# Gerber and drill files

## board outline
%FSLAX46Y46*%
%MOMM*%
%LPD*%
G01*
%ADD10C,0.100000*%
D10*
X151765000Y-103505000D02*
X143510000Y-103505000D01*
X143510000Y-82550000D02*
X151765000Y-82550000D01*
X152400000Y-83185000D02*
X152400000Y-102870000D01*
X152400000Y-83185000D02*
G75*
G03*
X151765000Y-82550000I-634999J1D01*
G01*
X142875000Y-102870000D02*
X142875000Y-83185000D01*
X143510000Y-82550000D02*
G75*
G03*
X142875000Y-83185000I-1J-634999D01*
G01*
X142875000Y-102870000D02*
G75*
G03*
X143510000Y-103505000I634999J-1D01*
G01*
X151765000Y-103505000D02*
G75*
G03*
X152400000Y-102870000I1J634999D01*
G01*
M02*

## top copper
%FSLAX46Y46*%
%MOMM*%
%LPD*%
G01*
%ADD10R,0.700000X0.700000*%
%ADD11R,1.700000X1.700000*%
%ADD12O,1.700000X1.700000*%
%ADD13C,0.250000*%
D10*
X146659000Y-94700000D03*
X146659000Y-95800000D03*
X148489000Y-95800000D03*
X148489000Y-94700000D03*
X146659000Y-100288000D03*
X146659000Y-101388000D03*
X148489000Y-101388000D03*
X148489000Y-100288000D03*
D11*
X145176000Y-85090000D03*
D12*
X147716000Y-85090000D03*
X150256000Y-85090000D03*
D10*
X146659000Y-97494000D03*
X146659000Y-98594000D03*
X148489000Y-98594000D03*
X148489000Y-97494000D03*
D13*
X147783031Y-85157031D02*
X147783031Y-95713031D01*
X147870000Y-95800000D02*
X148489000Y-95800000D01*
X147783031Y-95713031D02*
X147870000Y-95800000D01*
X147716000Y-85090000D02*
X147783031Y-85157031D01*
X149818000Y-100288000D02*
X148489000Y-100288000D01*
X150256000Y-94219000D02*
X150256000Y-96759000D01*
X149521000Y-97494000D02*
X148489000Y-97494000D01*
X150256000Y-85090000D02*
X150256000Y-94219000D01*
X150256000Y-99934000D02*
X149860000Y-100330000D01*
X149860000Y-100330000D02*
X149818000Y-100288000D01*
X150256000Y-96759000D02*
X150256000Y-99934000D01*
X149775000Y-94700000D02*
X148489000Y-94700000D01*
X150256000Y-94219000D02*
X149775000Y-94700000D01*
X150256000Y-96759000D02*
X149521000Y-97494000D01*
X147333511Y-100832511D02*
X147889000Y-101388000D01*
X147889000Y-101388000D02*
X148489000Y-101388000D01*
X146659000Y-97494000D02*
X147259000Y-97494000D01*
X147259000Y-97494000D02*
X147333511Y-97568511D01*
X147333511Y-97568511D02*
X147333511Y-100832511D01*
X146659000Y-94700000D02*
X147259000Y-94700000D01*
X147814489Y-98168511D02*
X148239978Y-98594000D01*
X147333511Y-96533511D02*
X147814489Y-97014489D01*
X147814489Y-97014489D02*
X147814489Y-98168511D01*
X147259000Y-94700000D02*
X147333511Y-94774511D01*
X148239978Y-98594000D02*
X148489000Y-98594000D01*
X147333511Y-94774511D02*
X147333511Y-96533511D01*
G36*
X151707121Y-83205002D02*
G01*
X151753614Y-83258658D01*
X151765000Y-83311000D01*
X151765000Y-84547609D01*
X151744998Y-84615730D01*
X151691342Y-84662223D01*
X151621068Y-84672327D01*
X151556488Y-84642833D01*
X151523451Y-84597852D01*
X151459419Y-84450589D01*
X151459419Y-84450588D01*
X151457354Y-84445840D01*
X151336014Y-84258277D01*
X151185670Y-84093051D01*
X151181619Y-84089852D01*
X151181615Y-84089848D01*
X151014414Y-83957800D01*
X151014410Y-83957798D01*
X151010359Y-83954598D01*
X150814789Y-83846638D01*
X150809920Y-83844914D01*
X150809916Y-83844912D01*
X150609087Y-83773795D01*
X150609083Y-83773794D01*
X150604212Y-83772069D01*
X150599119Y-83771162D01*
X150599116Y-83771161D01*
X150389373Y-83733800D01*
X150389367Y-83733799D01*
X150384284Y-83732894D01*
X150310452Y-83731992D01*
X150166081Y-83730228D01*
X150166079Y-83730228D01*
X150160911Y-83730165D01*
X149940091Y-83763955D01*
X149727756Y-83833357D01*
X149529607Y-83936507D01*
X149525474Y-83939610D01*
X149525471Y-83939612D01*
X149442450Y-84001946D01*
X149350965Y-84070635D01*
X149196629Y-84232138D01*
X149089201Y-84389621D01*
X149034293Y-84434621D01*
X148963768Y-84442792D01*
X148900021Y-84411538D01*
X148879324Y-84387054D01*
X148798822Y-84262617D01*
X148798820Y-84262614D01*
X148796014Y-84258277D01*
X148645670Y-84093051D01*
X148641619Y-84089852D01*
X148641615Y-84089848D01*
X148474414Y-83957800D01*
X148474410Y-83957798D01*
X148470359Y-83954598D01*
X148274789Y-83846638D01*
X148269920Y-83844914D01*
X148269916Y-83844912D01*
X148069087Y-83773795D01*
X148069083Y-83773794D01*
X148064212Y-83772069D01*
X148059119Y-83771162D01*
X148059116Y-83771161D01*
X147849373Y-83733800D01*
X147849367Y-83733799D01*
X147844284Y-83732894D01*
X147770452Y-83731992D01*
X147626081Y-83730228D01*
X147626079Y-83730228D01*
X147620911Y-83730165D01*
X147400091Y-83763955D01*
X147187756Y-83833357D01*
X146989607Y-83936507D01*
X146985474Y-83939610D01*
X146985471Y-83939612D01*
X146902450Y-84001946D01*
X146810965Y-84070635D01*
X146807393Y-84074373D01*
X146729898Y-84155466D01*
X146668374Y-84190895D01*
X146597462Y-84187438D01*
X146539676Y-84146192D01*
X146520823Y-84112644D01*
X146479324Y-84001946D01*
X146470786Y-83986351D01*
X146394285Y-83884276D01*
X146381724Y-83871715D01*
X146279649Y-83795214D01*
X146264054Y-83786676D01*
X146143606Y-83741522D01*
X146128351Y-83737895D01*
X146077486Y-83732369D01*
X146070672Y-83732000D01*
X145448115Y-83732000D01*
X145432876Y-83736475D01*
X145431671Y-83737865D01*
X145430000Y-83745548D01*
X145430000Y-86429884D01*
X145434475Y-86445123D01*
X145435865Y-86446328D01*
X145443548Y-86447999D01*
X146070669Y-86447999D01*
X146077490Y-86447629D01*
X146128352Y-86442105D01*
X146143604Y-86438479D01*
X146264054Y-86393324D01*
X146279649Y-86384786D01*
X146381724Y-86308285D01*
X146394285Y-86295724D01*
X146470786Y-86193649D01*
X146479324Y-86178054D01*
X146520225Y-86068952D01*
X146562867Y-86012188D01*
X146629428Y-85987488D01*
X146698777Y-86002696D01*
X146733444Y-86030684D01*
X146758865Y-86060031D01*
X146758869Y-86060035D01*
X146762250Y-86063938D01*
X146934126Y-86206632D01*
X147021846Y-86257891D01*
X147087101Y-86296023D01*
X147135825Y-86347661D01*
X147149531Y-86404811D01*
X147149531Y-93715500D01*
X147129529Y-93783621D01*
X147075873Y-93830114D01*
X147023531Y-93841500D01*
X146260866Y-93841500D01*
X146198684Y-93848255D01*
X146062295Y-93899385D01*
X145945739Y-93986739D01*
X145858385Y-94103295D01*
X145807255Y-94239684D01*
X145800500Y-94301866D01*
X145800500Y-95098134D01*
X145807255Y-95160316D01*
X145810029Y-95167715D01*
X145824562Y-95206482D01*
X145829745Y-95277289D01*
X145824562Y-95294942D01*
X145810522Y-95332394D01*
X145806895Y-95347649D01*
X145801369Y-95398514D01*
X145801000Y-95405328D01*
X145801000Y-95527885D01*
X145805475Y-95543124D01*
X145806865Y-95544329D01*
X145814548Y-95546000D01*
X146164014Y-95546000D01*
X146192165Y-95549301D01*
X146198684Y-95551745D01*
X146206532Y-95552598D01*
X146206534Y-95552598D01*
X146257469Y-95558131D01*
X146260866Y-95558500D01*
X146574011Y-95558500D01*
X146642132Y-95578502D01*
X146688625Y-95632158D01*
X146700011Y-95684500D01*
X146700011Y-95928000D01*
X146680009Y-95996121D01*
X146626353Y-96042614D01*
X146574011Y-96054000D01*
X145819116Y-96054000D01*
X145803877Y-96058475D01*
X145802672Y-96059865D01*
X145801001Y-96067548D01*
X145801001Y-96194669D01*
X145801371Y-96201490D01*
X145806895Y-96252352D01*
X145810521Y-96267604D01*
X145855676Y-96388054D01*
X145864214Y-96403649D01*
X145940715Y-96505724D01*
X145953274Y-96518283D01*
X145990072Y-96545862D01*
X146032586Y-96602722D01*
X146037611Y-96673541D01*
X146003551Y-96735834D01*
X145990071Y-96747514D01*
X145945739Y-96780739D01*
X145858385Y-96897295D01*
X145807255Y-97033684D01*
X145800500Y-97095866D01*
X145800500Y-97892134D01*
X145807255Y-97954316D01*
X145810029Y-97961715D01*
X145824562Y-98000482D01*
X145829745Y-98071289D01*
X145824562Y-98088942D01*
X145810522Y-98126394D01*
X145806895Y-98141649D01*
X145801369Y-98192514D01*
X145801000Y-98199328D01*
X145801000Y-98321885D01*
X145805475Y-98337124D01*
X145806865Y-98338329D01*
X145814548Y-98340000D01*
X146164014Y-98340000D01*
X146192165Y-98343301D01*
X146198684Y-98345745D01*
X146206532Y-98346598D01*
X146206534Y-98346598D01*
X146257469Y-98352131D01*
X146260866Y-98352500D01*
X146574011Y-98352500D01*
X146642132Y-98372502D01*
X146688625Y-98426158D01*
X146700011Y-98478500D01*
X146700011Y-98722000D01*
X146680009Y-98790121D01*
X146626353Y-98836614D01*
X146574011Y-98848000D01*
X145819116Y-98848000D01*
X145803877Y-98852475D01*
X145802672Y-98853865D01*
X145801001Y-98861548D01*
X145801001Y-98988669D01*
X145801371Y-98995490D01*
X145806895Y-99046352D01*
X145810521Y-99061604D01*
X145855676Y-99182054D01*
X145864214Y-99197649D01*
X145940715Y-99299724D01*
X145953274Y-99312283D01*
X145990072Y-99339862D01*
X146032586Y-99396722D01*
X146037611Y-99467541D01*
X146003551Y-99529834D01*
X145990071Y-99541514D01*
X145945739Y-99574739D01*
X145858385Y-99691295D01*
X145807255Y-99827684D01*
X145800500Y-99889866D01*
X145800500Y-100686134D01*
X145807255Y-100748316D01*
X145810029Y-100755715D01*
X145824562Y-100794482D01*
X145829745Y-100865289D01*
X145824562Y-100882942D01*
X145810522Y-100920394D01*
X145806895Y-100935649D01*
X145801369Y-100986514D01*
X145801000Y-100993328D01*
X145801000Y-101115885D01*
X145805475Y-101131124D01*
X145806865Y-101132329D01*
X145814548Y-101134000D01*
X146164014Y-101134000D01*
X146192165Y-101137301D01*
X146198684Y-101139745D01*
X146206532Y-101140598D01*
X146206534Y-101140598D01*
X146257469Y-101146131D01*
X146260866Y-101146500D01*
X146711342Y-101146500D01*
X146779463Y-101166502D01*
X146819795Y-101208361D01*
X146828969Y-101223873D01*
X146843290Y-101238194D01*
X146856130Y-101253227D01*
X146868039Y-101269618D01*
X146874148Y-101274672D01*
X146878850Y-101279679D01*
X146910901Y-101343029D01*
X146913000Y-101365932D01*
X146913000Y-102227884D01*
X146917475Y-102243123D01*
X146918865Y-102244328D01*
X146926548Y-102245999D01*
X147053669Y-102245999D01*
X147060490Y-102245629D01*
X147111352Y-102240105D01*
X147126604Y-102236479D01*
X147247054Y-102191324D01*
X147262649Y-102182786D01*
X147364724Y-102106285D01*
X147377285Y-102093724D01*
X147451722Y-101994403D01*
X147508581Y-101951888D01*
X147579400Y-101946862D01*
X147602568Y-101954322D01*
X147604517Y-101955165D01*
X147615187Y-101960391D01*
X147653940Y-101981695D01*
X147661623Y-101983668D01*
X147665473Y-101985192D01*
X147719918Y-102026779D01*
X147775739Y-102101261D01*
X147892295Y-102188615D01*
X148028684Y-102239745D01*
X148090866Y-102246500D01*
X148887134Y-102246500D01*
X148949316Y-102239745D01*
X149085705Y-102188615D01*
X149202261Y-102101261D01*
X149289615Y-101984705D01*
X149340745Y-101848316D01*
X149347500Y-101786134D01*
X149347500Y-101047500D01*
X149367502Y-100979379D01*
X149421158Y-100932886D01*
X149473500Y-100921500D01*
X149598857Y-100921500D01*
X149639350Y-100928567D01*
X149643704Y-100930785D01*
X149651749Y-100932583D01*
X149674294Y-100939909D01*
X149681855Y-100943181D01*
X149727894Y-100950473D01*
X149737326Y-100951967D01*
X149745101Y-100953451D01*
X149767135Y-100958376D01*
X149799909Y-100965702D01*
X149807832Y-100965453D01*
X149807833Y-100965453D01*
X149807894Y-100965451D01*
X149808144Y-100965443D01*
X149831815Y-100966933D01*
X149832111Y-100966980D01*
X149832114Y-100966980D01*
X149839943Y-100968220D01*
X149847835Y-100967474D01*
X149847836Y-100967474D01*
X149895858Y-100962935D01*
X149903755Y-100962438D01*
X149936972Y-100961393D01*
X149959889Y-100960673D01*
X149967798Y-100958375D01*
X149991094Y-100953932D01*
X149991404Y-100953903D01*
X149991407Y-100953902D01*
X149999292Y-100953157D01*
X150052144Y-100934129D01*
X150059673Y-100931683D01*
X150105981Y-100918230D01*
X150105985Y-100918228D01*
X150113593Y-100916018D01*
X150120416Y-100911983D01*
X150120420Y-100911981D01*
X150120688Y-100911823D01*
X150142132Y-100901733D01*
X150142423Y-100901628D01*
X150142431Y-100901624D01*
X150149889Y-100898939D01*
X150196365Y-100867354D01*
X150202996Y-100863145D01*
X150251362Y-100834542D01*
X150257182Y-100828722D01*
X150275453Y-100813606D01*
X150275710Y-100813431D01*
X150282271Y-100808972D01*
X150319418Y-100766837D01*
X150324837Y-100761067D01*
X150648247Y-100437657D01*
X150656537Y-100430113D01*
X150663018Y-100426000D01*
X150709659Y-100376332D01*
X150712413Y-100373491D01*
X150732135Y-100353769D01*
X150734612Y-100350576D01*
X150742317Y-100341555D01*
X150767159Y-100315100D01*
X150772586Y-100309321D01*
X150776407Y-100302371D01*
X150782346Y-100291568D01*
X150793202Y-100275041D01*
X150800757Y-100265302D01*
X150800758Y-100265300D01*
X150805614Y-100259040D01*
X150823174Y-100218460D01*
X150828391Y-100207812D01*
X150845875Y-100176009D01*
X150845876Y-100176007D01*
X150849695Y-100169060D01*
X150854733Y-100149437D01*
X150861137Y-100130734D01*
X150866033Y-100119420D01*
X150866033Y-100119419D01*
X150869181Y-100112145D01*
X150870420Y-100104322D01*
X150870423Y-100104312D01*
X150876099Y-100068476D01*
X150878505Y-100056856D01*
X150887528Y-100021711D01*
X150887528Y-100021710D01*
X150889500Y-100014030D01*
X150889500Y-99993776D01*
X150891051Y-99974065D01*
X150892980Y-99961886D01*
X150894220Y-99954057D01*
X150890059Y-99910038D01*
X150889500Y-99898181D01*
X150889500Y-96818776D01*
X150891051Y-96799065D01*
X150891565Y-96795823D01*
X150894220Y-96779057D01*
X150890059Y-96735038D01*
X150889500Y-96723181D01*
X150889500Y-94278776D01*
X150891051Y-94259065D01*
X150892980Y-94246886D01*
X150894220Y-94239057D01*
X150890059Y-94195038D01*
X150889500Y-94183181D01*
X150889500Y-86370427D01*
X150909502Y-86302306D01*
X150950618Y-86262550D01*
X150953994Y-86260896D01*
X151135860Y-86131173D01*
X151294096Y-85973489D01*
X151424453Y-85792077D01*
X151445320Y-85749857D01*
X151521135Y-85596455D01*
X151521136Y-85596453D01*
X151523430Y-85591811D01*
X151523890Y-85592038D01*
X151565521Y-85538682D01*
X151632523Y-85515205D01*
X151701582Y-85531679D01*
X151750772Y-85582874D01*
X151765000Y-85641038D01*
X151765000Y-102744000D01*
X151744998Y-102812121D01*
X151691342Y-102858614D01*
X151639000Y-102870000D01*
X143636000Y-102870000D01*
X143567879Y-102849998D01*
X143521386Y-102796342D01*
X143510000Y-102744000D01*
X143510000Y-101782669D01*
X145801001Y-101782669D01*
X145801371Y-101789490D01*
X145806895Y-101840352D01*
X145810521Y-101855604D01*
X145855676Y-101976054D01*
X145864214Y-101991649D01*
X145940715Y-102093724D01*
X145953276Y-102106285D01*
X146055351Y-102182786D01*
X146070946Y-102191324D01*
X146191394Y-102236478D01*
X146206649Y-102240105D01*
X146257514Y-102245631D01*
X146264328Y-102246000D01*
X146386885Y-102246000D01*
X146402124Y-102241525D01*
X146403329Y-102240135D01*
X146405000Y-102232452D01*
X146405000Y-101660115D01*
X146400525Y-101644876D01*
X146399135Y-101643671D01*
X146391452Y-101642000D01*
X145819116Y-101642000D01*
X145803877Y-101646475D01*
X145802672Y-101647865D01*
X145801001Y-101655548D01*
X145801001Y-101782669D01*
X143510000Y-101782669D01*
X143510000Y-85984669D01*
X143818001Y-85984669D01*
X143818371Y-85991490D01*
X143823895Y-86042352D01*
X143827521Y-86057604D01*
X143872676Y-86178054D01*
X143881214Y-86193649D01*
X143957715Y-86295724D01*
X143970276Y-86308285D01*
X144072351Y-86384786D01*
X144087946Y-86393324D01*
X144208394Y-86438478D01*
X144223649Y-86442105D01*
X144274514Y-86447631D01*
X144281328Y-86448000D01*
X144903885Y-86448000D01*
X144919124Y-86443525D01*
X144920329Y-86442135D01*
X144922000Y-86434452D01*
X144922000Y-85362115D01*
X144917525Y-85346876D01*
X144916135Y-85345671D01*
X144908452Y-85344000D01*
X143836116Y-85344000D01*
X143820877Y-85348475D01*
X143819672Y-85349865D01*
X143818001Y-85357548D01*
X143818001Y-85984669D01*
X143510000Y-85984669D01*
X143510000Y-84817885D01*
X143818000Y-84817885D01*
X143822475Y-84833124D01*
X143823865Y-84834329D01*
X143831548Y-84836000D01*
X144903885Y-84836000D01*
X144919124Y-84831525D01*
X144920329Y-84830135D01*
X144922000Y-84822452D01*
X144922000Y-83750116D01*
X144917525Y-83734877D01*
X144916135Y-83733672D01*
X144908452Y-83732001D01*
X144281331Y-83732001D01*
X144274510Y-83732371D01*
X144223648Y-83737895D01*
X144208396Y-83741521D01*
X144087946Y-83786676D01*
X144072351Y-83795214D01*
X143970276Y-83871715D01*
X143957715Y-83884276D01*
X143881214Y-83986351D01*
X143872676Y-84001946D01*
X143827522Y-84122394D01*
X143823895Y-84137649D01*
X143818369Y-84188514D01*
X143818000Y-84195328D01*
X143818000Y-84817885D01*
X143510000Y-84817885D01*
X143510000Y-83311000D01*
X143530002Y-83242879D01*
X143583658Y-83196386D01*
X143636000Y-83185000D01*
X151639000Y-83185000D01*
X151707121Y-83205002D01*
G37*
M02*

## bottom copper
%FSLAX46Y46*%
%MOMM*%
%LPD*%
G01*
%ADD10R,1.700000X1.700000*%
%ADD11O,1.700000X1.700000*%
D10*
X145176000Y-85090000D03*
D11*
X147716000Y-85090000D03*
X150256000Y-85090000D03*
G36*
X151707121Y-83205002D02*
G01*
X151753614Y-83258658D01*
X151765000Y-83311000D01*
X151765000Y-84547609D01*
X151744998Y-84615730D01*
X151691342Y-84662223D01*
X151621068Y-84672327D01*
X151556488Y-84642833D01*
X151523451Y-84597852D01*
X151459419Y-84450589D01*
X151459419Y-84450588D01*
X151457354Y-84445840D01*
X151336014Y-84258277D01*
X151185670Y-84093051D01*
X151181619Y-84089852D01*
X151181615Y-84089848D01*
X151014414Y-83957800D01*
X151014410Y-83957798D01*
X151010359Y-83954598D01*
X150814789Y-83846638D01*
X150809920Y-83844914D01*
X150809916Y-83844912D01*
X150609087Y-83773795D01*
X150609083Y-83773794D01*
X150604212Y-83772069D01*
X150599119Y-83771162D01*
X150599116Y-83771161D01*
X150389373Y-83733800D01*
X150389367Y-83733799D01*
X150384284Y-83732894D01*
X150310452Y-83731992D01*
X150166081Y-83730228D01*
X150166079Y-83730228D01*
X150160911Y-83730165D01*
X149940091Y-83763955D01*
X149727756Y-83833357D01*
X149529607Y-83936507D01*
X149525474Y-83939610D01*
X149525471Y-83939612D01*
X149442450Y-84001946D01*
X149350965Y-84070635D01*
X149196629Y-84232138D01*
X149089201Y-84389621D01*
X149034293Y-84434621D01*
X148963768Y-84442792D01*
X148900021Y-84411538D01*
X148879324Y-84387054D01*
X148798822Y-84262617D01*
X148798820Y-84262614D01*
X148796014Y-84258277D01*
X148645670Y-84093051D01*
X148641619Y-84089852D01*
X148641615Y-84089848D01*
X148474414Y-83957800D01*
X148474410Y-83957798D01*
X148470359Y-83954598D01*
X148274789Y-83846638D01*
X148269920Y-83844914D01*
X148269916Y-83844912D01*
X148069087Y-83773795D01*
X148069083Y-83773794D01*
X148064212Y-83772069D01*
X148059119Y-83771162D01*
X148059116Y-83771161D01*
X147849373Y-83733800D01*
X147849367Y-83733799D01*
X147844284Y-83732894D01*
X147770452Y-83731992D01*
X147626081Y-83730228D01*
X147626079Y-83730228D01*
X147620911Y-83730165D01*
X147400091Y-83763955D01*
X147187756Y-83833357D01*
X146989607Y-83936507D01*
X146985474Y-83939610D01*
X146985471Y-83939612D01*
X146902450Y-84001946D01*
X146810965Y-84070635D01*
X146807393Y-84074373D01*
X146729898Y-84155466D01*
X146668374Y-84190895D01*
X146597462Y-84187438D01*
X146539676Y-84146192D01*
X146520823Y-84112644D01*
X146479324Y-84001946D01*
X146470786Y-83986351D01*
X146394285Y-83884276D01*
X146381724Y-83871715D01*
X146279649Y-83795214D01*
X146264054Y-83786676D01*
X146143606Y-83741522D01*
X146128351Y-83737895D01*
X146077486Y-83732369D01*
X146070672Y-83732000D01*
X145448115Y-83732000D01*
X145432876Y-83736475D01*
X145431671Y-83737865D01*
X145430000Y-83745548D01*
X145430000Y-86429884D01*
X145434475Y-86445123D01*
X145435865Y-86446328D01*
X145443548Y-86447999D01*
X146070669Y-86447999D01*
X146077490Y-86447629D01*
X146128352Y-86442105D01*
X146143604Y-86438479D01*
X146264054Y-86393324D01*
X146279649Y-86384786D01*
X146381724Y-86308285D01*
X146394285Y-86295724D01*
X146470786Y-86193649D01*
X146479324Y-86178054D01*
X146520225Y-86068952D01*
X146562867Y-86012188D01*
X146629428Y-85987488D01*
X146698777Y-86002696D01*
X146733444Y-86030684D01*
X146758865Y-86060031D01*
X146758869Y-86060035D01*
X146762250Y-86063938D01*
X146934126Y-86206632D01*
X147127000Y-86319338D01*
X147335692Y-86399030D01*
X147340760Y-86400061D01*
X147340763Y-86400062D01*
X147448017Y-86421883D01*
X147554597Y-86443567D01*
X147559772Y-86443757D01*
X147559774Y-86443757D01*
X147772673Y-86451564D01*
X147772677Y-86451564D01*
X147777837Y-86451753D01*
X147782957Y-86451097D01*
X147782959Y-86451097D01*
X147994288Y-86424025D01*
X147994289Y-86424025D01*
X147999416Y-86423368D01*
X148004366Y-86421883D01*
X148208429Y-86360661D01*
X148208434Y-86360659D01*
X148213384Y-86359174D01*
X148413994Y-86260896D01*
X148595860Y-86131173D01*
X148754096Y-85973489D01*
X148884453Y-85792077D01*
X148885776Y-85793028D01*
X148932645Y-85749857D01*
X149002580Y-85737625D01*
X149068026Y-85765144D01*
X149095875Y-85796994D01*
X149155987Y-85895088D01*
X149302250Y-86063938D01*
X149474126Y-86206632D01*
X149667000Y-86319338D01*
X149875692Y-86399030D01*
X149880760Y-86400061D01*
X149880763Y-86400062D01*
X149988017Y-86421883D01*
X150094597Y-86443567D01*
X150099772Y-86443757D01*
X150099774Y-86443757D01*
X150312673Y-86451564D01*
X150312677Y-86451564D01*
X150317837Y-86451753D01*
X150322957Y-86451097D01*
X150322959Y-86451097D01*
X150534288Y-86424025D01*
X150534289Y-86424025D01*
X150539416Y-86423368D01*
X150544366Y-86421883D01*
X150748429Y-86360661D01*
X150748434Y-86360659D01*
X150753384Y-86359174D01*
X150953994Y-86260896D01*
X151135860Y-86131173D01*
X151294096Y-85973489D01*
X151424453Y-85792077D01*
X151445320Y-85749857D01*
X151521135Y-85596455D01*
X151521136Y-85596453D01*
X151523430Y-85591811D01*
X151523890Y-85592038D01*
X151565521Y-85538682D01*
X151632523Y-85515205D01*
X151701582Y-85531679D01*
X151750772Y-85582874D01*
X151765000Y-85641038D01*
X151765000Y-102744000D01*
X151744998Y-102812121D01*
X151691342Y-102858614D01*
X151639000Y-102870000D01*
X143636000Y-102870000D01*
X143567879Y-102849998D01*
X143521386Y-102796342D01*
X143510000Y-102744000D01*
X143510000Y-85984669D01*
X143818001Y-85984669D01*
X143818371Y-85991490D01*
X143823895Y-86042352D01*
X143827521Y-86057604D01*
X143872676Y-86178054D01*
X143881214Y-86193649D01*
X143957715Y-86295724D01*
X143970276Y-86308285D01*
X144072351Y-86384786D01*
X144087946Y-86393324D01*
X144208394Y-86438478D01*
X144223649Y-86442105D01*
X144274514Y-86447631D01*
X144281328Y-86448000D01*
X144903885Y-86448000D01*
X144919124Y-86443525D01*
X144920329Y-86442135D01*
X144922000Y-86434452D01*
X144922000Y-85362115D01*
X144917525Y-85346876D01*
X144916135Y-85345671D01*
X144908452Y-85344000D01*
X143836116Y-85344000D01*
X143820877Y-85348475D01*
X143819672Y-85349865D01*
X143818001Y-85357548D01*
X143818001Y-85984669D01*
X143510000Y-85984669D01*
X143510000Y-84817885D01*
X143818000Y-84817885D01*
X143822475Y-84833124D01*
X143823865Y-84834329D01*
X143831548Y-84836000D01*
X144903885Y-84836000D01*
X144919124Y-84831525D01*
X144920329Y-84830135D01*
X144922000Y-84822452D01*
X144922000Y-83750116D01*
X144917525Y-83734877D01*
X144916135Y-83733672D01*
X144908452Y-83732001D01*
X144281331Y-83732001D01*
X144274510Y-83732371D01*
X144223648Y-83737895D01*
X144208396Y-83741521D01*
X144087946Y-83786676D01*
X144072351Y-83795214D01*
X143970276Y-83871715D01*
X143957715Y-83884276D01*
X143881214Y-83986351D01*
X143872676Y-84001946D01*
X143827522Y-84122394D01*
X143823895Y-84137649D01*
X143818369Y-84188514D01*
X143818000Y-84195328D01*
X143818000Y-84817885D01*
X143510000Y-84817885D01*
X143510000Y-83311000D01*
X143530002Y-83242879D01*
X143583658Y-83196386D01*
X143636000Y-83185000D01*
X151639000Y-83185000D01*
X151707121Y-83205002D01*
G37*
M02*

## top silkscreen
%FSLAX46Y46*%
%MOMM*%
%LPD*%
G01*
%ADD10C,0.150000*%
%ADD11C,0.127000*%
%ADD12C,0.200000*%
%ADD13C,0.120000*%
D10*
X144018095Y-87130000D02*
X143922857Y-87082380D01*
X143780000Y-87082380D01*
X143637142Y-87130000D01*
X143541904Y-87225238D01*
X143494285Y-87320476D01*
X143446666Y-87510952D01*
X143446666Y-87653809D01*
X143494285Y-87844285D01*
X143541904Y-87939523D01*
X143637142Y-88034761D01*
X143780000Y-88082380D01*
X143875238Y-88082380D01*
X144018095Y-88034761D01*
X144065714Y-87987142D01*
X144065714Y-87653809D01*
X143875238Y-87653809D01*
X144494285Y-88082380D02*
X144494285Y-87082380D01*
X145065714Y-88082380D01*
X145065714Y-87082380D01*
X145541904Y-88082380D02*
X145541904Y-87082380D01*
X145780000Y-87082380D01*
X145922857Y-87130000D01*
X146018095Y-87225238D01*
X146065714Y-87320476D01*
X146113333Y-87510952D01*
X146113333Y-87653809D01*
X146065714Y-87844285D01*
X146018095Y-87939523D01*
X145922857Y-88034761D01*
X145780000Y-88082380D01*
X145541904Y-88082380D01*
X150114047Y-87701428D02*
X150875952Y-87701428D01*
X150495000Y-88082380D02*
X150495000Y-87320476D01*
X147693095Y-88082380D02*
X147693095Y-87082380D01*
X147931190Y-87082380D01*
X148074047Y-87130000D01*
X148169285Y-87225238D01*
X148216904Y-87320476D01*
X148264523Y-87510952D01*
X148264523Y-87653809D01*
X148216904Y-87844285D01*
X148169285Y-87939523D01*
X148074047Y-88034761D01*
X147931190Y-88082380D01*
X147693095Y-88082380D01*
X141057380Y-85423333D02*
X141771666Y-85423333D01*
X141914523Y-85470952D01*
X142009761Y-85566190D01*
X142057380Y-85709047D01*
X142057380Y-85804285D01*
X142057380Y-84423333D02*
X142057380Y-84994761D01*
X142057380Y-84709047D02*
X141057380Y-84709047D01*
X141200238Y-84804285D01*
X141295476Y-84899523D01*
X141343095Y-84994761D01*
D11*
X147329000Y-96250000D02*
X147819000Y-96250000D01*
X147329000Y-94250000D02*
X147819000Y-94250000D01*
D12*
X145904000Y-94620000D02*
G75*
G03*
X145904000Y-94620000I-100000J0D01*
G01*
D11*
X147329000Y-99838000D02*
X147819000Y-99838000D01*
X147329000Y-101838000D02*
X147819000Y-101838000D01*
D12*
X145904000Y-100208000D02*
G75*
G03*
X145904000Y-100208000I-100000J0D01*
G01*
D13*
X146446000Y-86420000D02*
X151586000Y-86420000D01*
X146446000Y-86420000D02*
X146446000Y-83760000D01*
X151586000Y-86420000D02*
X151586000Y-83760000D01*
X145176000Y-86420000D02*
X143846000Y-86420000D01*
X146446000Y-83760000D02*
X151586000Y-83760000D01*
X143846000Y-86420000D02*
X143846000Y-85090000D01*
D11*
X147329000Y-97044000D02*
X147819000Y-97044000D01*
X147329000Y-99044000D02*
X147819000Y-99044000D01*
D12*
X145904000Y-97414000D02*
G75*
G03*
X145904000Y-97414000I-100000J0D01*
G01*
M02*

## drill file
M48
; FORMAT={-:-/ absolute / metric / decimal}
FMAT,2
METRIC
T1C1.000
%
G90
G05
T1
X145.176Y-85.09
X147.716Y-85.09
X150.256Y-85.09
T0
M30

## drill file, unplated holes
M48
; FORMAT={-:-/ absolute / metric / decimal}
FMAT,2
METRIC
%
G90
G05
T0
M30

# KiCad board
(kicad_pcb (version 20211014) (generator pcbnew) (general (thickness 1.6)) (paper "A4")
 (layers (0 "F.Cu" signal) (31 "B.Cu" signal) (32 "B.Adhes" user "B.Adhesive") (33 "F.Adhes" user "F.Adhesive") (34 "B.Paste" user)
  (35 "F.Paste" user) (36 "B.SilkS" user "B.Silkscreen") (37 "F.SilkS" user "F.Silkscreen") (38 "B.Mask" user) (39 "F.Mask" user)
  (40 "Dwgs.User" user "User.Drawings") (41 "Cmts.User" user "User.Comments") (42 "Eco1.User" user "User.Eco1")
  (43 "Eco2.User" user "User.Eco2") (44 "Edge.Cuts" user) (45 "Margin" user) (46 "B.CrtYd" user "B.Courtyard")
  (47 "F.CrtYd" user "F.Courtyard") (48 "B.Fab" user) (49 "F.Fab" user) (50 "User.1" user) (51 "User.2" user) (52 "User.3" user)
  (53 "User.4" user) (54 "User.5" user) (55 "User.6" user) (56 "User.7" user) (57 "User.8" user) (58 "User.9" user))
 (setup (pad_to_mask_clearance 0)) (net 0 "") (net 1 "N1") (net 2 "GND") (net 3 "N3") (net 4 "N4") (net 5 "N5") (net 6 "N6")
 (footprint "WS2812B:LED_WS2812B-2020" (layer "F.Cu") (at 147.574 95.25)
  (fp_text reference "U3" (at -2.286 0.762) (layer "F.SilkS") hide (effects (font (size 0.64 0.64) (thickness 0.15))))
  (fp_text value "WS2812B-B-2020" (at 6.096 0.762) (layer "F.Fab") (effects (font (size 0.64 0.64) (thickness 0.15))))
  (fp_line (start -0.245 1) (end 0.245 1) (layer "F.SilkS") (width 0.127))
  (fp_line (start -0.245 -1) (end 0.245 -1) (layer "F.SilkS") (width 0.127))
  (fp_circle (center -1.77 -0.63) (end -1.67 -0.63) (layer "F.SilkS") (width 0.2) (fill none))
  (pad "1" smd rect (at -0.915 -0.55) (size 0.7 0.7) (layers "F.Cu" "F.Paste" "F.Mask") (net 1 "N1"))
  (pad "2" smd rect (at -0.915 0.55) (size 0.7 0.7) (layers "F.Cu" "F.Paste" "F.Mask") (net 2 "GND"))
  (pad "3" smd rect (at 0.915 0.55) (size 0.7 0.7) (layers "F.Cu" "F.Paste" "F.Mask") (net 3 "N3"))
  (pad "4" smd rect (at 0.915 -0.55) (size 0.7 0.7) (layers "F.Cu" "F.Paste" "F.Mask") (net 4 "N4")))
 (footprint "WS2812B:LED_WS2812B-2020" (layer "F.Cu") (at 147.574 100.838)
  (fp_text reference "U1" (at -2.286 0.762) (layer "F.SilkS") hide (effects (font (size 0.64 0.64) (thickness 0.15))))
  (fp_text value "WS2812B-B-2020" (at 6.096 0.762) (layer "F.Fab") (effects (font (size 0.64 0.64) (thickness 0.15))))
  (fp_line (start -0.245 -1) (end 0.245 -1) (layer "F.SilkS") (width 0.127))
  (fp_line (start -0.245 1) (end 0.245 1) (layer "F.SilkS") (width 0.127))
  (fp_circle (center -1.77 -0.63) (end -1.67 -0.63) (layer "F.SilkS") (width 0.2) (fill none))
  (pad "1" smd rect (at -0.915 -0.55) (size 0.7 0.7) (layers "F.Cu" "F.Paste" "F.Mask") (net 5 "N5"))
  (pad "2" smd rect (at -0.915 0.55) (size 0.7 0.7) (layers "F.Cu" "F.Paste" "F.Mask") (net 2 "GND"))
  (pad "3" smd rect (at 0.915 0.55) (size 0.7 0.7) (layers "F.Cu" "F.Paste" "F.Mask") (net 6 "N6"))
  (pad "4" smd rect (at 0.915 -0.55) (size 0.7 0.7) (layers "F.Cu" "F.Paste" "F.Mask") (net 4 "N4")))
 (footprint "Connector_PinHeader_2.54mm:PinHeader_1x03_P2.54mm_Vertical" (layer "F.Cu") (at 145.176 85.09 90)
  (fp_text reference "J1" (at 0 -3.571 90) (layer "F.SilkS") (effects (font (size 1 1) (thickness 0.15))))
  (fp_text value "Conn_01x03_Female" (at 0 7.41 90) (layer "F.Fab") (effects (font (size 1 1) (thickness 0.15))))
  (fp_line (start -1.33 1.27) (end -1.33 6.41) (layer "F.SilkS") (width 0.12))
  (fp_line (start -1.33 1.27) (end 1.33 1.27) (layer "F.SilkS") (width 0.12))
  (fp_line (start -1.33 6.41) (end 1.33 6.41) (layer "F.SilkS") (width 0.12))
  (fp_line (start -1.33 0) (end -1.33 -1.33) (layer "F.SilkS") (width 0.12))
  (fp_line (start 1.33 1.27) (end 1.33 6.41) (layer "F.SilkS") (width 0.12))
  (fp_line (start -1.33 -1.33) (end 0 -1.33) (layer "F.SilkS") (width 0.12))
  (pad "1" thru_hole rect (at 0 0 90) (size 1.7 1.7) (drill 1) (layers *.Cu *.Mask) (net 2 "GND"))
  (pad "2" thru_hole oval (at 0 2.54 90) (size 1.7 1.7) (drill 1) (layers *.Cu *.Mask) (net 3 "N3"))
  (pad "3" thru_hole oval (at 0 5.08 90) (size 1.7 1.7) (drill 1) (layers *.Cu *.Mask) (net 4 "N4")))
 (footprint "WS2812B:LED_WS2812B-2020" (layer "F.Cu") (at 147.574 98.044)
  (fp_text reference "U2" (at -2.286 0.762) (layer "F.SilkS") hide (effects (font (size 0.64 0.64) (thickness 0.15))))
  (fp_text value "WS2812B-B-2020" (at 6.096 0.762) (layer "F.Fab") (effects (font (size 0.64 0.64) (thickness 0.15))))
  (fp_line (start -0.245 -1) (end 0.245 -1) (layer "F.SilkS") (width 0.127))
  (fp_line (start -0.245 1) (end 0.245 1) (layer "F.SilkS") (width 0.127))
  (fp_circle (center -1.77 -0.63) (end -1.67 -0.63) (layer "F.SilkS") (width 0.2) (fill none))
  (pad "1" smd rect (at -0.915 -0.55) (size 0.7 0.7) (layers "F.Cu" "F.Paste" "F.Mask") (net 6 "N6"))
  (pad "2" smd rect (at -0.915 0.55) (size 0.7 0.7) (layers "F.Cu" "F.Paste" "F.Mask") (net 2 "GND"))
  (pad "3" smd rect (at 0.915 0.55) (size 0.7 0.7) (layers "F.Cu" "F.Paste" "F.Mask") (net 1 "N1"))
  (pad "4" smd rect (at 0.915 -0.55) (size 0.7 0.7) (layers "F.Cu" "F.Paste" "F.Mask") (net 4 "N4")))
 (gr_line (start 151.765 103.505) (end 143.51 103.505) (layer "Edge.Cuts") (width 0.1))
 (gr_line (start 143.51 82.55) (end 151.765 82.55) (layer "Edge.Cuts") (width 0.1))
 (gr_line (start 152.4 83.185) (end 152.4 102.87) (layer "Edge.Cuts") (width 0.1))
 (gr_arc (start 151.765 82.55) (mid 152.214013 82.735987) (end 152.4 83.185) (layer "Edge.Cuts") (width 0.1))
 (gr_line (start 142.875 102.87) (end 142.875 83.185) (layer "Edge.Cuts") (width 0.1))
 (gr_arc (start 142.875 83.185) (mid 143.060987 82.735987) (end 143.51 82.55) (layer "Edge.Cuts") (width 0.1))
 (gr_arc (start 143.51 103.505) (mid 143.060987 103.319013) (end 142.875 102.87) (layer "Edge.Cuts") (width 0.1))
 (gr_arc (start 152.4 102.87) (mid 152.214013 103.319013) (end 151.765 103.505) (layer "Edge.Cuts") (width 0.1))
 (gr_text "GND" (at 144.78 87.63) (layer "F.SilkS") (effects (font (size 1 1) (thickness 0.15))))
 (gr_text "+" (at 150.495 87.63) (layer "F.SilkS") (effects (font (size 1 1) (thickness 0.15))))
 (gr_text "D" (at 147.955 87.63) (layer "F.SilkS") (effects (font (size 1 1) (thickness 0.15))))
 (segment (start 147.783031 85.157031) (end 147.783031 95.713031) (width 0.25) (layer "F.Cu") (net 3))
 (segment (start 147.87 95.8) (end 148.489 95.8) (width 0.25) (layer "F.Cu") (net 3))
 (segment (start 147.783031 95.713031) (end 147.87 95.8) (width 0.25) (layer "F.Cu") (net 3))
 (segment (start 147.716 85.09) (end 147.783031 85.157031) (width 0.25) (layer "F.Cu") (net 3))
 (segment (start 149.818 100.288) (end 148.489 100.288) (width 0.25) (layer "F.Cu") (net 4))
 (segment (start 150.256 94.219) (end 150.256 96.759) (width 0.25) (layer "F.Cu") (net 4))
 (segment (start 149.521 97.494) (end 148.489 97.494) (width 0.25) (layer "F.Cu") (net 4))
 (segment (start 150.256 85.09) (end 150.256 94.219) (width 0.25) (layer "F.Cu") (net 4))
 (segment (start 150.256 99.934) (end 149.86 100.33) (width 0.25) (layer "F.Cu") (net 4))
 (segment (start 149.86 100.33) (end 149.818 100.288) (width 0.25) (layer "F.Cu") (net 4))
 (segment (start 150.256 96.759) (end 150.256 99.934) (width 0.25) (layer "F.Cu") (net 4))
 (segment (start 149.775 94.7) (end 148.489 94.7) (width 0.25) (layer "F.Cu") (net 4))
 (segment (start 150.256 94.219) (end 149.775 94.7) (width 0.25) (layer "F.Cu") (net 4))
 (segment (start 150.256 96.759) (end 149.521 97.494) (width 0.25) (layer "F.Cu") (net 4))
 (segment (start 147.333511 100.832511) (end 147.889 101.388) (width 0.25) (layer "F.Cu") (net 6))
 (segment (start 147.889 101.388) (end 148.489 101.388) (width 0.25) (layer "F.Cu") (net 6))
 (segment (start 146.659 97.494) (end 147.259 97.494) (width 0.25) (layer "F.Cu") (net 6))
 (segment (start 147.259 97.494) (end 147.333511 97.568511) (width 0.25) (layer "F.Cu") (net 6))
 (segment (start 147.333511 97.568511) (end 147.333511 100.832511) (width 0.25) (layer "F.Cu") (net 6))
 (segment (start 146.659 94.7) (end 147.259 94.7) (width 0.25) (layer "F.Cu") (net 1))
 (segment (start 147.814489 98.168511) (end 148.239978 98.594) (width 0.25) (layer "F.Cu") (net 1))
 (segment (start 147.333511 96.533511) (end 147.814489 97.014489) (width 0.25) (layer "F.Cu") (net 1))
 (segment (start 147.814489 97.014489) (end 147.814489 98.168511) (width 0.25) (layer "F.Cu") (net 1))
 (segment (start 147.259 94.7) (end 147.333511 94.774511) (width 0.25) (layer "F.Cu") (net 1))
 (segment (start 148.239978 98.594) (end 148.489 98.594) (width 0.25) (layer "F.Cu") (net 1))
 (segment (start 147.333511 94.774511) (end 147.333511 96.533511) (width 0.25) (layer "F.Cu") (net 1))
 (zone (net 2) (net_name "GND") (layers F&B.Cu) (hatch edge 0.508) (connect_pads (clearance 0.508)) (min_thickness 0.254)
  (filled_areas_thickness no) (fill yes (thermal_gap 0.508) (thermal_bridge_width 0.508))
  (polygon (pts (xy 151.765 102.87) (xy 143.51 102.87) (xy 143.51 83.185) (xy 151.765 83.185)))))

